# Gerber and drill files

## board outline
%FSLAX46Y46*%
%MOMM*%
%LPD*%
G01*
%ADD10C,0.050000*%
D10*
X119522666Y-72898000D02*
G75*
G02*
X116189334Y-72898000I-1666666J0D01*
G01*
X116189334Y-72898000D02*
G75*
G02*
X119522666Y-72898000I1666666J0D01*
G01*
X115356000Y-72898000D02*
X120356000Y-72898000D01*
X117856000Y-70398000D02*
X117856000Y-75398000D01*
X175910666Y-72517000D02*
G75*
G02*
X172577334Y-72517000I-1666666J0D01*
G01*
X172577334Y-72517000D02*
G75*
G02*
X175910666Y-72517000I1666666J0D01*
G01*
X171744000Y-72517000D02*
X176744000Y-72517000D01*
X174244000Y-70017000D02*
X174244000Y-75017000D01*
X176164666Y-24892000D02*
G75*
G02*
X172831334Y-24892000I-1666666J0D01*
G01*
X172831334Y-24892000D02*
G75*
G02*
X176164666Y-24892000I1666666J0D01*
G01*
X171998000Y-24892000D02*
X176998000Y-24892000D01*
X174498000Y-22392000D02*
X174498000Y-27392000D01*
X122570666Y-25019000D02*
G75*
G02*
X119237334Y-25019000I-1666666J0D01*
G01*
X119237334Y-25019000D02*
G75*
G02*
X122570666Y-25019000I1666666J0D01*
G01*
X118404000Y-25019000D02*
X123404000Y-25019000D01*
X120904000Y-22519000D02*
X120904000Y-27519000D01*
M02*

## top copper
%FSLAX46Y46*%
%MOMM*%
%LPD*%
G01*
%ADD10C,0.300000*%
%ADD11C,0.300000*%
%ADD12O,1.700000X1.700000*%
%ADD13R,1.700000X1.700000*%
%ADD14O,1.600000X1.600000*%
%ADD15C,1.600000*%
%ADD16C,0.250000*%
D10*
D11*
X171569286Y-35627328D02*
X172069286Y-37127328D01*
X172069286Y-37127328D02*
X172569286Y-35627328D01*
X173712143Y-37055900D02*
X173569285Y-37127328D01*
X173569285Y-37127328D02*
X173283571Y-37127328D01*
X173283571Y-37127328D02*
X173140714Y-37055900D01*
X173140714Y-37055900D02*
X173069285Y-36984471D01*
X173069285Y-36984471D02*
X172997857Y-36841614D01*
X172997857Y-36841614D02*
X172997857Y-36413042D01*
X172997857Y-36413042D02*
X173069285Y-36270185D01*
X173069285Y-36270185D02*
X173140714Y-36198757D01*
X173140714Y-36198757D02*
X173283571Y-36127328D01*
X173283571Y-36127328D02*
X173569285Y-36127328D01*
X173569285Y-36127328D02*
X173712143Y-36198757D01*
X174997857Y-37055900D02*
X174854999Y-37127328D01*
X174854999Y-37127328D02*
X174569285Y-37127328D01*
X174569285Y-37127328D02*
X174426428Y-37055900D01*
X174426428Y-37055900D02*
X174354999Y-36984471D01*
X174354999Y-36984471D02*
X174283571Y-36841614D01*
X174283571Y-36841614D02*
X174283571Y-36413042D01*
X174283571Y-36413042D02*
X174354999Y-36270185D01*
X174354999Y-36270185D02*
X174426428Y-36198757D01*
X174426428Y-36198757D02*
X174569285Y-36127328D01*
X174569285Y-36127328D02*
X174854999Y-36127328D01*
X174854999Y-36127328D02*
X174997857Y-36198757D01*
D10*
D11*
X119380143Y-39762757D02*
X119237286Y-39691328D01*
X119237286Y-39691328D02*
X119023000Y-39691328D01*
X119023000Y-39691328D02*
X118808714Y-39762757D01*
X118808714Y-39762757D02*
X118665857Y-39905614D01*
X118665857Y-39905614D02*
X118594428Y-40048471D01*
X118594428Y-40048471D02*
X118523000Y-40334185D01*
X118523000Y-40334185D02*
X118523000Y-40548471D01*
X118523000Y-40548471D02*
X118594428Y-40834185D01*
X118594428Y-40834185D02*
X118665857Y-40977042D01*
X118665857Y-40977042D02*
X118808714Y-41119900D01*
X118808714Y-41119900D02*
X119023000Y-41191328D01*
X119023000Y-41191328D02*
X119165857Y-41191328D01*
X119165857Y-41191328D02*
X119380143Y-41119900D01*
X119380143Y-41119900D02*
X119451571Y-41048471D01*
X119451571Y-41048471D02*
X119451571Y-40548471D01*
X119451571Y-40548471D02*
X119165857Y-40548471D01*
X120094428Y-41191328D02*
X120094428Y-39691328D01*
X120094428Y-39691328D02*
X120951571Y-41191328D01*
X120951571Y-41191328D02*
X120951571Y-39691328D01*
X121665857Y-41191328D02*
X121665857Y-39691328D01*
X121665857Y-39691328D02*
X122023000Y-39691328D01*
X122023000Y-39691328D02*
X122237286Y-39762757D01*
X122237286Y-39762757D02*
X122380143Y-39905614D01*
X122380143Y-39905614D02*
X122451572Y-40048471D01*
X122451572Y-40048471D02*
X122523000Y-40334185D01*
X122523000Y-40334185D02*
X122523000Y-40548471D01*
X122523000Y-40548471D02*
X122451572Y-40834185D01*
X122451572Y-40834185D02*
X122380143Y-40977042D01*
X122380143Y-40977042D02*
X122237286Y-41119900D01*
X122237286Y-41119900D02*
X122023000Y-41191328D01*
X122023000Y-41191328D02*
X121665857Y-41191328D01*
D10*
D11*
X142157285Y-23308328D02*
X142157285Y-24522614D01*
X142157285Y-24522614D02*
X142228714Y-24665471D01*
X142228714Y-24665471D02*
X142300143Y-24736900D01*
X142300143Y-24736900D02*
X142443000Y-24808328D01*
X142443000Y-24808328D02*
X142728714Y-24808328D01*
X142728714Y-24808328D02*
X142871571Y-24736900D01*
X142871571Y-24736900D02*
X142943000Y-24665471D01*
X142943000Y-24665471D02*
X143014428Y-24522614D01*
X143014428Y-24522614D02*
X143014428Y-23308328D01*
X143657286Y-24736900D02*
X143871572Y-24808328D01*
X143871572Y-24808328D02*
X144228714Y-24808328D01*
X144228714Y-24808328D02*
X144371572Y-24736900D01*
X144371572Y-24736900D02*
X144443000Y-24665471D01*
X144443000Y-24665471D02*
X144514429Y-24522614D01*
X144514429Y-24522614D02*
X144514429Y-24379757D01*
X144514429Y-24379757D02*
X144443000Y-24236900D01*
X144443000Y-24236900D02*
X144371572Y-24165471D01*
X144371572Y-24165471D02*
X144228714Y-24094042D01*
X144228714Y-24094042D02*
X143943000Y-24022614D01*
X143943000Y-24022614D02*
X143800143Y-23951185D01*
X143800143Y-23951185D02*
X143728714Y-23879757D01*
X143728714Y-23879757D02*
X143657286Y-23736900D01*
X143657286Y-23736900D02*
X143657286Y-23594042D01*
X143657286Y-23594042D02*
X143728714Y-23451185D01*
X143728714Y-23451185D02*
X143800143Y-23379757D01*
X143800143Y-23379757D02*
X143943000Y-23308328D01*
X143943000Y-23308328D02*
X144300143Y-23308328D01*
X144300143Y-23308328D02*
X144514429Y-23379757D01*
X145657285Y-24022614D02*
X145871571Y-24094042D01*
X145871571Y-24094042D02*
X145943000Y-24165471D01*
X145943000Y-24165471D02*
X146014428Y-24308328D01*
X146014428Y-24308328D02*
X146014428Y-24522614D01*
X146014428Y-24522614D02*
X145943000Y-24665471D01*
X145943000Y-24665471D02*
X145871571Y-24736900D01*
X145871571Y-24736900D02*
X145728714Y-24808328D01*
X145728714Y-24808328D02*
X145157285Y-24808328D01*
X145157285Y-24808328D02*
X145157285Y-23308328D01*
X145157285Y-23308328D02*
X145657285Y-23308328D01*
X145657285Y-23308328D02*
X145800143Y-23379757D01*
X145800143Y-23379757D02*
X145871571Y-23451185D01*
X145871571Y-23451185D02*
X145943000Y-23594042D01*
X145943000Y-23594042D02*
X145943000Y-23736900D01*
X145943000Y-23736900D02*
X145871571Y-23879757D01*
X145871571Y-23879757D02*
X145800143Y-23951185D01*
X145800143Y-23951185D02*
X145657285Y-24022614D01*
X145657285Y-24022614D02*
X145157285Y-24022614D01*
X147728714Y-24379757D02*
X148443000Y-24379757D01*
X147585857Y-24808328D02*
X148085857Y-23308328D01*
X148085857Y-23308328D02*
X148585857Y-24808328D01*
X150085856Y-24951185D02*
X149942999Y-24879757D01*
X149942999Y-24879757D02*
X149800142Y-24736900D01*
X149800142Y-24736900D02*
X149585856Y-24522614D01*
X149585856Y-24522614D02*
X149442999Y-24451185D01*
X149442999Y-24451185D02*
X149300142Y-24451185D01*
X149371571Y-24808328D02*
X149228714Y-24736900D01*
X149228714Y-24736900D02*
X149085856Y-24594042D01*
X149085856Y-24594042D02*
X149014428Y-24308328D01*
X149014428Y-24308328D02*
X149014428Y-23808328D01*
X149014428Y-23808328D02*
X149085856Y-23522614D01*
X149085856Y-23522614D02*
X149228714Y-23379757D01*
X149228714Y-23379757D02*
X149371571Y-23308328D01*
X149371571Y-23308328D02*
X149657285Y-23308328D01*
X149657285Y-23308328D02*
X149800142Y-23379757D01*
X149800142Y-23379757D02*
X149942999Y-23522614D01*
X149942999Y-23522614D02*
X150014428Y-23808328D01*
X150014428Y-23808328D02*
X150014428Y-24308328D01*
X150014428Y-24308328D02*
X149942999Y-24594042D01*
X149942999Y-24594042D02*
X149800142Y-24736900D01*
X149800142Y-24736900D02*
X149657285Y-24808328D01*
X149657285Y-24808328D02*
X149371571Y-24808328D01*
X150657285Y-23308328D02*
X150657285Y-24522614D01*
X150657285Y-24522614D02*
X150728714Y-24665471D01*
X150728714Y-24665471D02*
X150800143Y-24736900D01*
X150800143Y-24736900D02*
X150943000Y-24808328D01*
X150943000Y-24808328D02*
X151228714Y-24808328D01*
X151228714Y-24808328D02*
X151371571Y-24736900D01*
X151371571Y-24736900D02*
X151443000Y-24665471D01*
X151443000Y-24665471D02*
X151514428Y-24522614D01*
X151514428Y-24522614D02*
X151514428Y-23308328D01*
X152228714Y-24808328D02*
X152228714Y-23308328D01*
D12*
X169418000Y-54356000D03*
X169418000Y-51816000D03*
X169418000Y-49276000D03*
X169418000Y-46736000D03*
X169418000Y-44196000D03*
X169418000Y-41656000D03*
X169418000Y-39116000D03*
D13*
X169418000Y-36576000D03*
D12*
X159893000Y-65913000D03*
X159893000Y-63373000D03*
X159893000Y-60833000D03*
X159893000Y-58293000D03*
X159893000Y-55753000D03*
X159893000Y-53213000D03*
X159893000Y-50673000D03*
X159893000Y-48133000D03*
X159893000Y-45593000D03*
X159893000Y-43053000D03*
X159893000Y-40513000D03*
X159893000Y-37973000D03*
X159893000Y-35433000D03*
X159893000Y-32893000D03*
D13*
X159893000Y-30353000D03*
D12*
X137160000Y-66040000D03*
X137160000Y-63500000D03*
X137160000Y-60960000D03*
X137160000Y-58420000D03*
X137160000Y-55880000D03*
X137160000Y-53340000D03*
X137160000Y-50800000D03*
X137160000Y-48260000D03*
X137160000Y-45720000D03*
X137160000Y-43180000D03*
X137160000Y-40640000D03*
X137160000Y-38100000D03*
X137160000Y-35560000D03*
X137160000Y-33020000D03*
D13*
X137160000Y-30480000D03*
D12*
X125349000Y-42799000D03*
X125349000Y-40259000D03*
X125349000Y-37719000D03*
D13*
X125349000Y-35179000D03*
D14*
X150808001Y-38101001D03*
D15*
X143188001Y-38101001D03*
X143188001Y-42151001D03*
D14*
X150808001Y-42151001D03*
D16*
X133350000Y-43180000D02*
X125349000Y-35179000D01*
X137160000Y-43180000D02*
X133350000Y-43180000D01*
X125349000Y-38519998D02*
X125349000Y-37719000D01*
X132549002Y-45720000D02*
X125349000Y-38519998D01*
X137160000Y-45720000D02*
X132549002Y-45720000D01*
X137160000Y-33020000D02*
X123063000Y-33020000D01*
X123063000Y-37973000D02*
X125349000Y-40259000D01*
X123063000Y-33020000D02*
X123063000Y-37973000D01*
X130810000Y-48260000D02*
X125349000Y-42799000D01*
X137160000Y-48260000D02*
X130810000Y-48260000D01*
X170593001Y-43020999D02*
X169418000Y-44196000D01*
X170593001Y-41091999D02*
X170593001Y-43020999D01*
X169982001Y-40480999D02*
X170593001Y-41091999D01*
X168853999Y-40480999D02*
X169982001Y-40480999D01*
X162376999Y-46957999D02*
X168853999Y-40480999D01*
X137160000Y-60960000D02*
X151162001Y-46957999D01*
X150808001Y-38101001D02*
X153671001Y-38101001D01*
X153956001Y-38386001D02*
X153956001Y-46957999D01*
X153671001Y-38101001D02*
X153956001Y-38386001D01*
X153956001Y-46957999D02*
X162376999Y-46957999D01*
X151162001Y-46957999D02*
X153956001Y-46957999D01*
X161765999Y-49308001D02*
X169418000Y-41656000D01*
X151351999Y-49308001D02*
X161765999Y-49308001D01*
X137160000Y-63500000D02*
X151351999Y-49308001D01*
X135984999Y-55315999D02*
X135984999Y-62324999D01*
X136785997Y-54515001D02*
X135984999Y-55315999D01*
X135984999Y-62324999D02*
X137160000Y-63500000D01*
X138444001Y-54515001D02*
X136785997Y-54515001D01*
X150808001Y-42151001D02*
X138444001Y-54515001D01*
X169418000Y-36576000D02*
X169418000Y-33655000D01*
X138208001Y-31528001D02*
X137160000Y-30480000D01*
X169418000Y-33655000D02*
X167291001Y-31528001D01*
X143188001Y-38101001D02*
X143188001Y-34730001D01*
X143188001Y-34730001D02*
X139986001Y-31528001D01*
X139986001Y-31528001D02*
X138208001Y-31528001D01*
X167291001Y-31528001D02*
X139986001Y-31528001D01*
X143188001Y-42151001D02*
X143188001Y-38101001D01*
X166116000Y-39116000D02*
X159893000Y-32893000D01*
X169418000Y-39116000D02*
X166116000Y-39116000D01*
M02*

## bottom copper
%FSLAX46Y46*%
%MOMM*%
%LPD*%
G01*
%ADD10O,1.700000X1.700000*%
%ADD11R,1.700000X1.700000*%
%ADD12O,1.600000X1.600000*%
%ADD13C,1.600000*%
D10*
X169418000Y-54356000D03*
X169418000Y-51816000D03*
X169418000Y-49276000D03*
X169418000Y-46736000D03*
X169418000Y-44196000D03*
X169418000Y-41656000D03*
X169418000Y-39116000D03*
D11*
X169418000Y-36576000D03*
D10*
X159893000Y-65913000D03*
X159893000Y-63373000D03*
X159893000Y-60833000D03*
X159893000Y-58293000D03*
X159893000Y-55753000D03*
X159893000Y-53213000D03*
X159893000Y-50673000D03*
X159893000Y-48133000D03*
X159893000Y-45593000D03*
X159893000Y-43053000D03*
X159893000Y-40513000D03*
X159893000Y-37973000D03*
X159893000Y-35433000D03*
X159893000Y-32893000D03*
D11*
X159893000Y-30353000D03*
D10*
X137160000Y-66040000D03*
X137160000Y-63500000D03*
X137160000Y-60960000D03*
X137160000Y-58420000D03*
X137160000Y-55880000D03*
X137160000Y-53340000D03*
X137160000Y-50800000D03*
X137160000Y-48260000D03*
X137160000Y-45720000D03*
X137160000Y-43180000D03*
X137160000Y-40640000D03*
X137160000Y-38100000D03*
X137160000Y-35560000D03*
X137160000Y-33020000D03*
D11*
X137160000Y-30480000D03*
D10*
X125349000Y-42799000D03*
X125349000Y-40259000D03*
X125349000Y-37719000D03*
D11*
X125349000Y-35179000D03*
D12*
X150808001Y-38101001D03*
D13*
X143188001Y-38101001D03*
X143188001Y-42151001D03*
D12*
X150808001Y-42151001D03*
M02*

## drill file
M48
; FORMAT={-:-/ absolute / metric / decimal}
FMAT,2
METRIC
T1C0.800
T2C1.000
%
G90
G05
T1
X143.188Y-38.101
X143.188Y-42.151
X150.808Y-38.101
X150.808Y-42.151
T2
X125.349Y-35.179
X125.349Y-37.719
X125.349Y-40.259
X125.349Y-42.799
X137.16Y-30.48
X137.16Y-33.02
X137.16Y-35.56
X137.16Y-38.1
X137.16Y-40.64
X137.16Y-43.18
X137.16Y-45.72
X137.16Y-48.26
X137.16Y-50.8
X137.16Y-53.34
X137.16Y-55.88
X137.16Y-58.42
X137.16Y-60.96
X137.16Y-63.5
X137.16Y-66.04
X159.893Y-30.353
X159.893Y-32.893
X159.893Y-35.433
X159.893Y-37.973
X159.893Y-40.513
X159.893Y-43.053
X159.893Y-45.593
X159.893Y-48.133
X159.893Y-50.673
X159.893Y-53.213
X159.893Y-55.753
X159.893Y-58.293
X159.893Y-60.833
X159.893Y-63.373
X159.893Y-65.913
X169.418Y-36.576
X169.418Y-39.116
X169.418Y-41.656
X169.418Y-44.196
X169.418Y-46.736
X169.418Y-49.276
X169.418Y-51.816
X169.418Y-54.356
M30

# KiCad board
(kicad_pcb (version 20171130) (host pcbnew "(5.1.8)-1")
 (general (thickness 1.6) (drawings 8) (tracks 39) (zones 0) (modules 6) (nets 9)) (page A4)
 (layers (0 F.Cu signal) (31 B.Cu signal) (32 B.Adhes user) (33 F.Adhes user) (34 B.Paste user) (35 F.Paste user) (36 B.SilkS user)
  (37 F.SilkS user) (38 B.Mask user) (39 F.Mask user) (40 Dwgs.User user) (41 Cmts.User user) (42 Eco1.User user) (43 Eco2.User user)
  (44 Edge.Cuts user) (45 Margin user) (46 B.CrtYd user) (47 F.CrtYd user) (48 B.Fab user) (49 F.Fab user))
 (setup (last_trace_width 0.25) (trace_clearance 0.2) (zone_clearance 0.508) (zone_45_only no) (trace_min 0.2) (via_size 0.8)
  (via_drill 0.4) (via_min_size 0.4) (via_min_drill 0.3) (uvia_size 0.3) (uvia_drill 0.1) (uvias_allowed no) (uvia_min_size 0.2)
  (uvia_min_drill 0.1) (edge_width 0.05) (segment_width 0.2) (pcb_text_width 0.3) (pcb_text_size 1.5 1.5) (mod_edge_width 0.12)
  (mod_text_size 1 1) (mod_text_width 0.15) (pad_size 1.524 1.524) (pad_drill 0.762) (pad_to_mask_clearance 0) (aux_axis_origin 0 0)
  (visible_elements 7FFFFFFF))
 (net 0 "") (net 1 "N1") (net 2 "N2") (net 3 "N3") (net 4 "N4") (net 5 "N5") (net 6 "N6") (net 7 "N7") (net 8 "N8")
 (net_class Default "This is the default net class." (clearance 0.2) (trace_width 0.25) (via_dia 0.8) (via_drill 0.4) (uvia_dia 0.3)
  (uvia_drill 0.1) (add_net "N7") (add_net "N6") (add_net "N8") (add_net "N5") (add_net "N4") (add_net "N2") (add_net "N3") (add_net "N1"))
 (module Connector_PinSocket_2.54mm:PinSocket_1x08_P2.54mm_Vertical (layer F.Cu) (at 169.418 36.576)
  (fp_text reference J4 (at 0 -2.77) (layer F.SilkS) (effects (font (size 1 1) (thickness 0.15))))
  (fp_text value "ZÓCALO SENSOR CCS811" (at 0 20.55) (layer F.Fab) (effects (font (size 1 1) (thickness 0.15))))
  (pad 8 thru_hole oval (at 0 17.78) (size 1.7 1.7) (drill 1) (layers *.Cu *.Mask))
  (pad 7 thru_hole oval (at 0 15.24) (size 1.7 1.7) (drill 1) (layers *.Cu *.Mask))
  (pad 6 thru_hole oval (at 0 12.7) (size 1.7 1.7) (drill 1) (layers *.Cu *.Mask))
  (pad 5 thru_hole oval (at 0 10.16) (size 1.7 1.7) (drill 1) (layers *.Cu *.Mask) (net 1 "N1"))
  (pad 4 thru_hole oval (at 0 7.62) (size 1.7 1.7) (drill 1) (layers *.Cu *.Mask) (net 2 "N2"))
  (pad 3 thru_hole oval (at 0 5.08) (size 1.7 1.7) (drill 1) (layers *.Cu *.Mask) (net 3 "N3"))
  (pad 2 thru_hole oval (at 0 2.54) (size 1.7 1.7) (drill 1) (layers *.Cu *.Mask) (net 1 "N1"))
  (pad 1 thru_hole rect (at 0 0) (size 1.7 1.7) (drill 1) (layers *.Cu *.Mask) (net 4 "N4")))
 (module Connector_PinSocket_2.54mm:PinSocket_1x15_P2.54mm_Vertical (layer F.Cu) (at 159.893 30.353)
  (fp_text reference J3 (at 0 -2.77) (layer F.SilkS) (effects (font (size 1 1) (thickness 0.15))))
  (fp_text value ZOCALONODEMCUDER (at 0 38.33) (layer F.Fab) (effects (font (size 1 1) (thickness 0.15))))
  (pad 15 thru_hole oval (at 0 35.56) (size 1.7 1.7) (drill 1) (layers *.Cu *.Mask))
  (pad 14 thru_hole oval (at 0 33.02) (size 1.7 1.7) (drill 1) (layers *.Cu *.Mask))
  (pad 13 thru_hole oval (at 0 30.48) (size 1.7 1.7) (drill 1) (layers *.Cu *.Mask))
  (pad 12 thru_hole oval (at 0 27.94) (size 1.7 1.7) (drill 1) (layers *.Cu *.Mask))
  (pad 11 thru_hole oval (at 0 25.4) (size 1.7 1.7) (drill 1) (layers *.Cu *.Mask))
  (pad 10 thru_hole oval (at 0 22.86) (size 1.7 1.7) (drill 1) (layers *.Cu *.Mask))
  (pad 9 thru_hole oval (at 0 20.32) (size 1.7 1.7) (drill 1) (layers *.Cu *.Mask))
  (pad 8 thru_hole oval (at 0 17.78) (size 1.7 1.7) (drill 1) (layers *.Cu *.Mask))
  (pad 7 thru_hole oval (at 0 15.24) (size 1.7 1.7) (drill 1) (layers *.Cu *.Mask))
  (pad 6 thru_hole oval (at 0 12.7) (size 1.7 1.7) (drill 1) (layers *.Cu *.Mask))
  (pad 5 thru_hole oval (at 0 10.16) (size 1.7 1.7) (drill 1) (layers *.Cu *.Mask))
  (pad 4 thru_hole oval (at 0 7.62) (size 1.7 1.7) (drill 1) (layers *.Cu *.Mask))
  (pad 3 thru_hole oval (at 0 5.08) (size 1.7 1.7) (drill 1) (layers *.Cu *.Mask))
  (pad 2 thru_hole oval (at 0 2.54) (size 1.7 1.7) (drill 1) (layers *.Cu *.Mask) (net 1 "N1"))
  (pad 1 thru_hole rect (at 0 0) (size 1.7 1.7) (drill 1) (layers *.Cu *.Mask)))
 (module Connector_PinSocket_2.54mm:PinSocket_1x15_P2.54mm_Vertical (layer F.Cu) (at 137.16 30.48)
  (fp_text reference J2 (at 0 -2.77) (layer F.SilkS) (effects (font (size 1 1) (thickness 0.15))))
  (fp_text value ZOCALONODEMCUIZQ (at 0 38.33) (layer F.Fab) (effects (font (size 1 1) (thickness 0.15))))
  (pad 15 thru_hole oval (at 0 35.56) (size 1.7 1.7) (drill 1) (layers *.Cu *.Mask))
  (pad 14 thru_hole oval (at 0 33.02) (size 1.7 1.7) (drill 1) (layers *.Cu *.Mask) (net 3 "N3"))
  (pad 13 thru_hole oval (at 0 30.48) (size 1.7 1.7) (drill 1) (layers *.Cu *.Mask) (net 2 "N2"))
  (pad 12 thru_hole oval (at 0 27.94) (size 1.7 1.7) (drill 1) (layers *.Cu *.Mask))
  (pad 11 thru_hole oval (at 0 25.4) (size 1.7 1.7) (drill 1) (layers *.Cu *.Mask))
  (pad 10 thru_hole oval (at 0 22.86) (size 1.7 1.7) (drill 1) (layers *.Cu *.Mask))
  (pad 9 thru_hole oval (at 0 20.32) (size 1.7 1.7) (drill 1) (layers *.Cu *.Mask))
  (pad 8 thru_hole oval (at 0 17.78) (size 1.7 1.7) (drill 1) (layers *.Cu *.Mask) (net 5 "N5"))
  (pad 7 thru_hole oval (at 0 15.24) (size 1.7 1.7) (drill 1) (layers *.Cu *.Mask) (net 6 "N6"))
  (pad 6 thru_hole oval (at 0 12.7) (size 1.7 1.7) (drill 1) (layers *.Cu *.Mask) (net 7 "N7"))
  (pad 5 thru_hole oval (at 0 10.16) (size 1.7 1.7) (drill 1) (layers *.Cu *.Mask))
  (pad 4 thru_hole oval (at 0 7.62) (size 1.7 1.7) (drill 1) (layers *.Cu *.Mask))
  (pad 3 thru_hole oval (at 0 5.08) (size 1.7 1.7) (drill 1) (layers *.Cu *.Mask))
  (pad 2 thru_hole oval (at 0 2.54) (size 1.7 1.7) (drill 1) (layers *.Cu *.Mask) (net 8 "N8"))
  (pad 1 thru_hole rect (at 0 0) (size 1.7 1.7) (drill 1) (layers *.Cu *.Mask) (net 4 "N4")))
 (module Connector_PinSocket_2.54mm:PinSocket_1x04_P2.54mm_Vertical (layer F.Cu) (at 125.349 35.179)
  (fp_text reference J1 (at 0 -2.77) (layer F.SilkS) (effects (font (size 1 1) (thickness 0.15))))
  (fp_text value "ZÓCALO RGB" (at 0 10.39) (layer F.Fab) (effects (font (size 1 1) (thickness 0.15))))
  (pad 4 thru_hole oval (at 0 7.62) (size 1.7 1.7) (drill 1) (layers *.Cu *.Mask) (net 5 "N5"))
  (pad 3 thru_hole oval (at 0 5.08) (size 1.7 1.7) (drill 1) (layers *.Cu *.Mask) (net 8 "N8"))
  (pad 2 thru_hole oval (at 0 2.54) (size 1.7 1.7) (drill 1) (layers *.Cu *.Mask) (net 6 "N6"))
  (pad 1 thru_hole rect (at 0 0) (size 1.7 1.7) (drill 1) (layers *.Cu *.Mask) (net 7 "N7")))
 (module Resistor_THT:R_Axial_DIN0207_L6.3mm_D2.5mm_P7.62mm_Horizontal (layer F.Cu) (at 143.188001 38.101001)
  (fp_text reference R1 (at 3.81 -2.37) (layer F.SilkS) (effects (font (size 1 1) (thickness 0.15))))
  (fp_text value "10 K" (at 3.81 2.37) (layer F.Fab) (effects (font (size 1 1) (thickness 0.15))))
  (pad 2 thru_hole oval (at 7.62 0) (size 1.6 1.6) (drill 0.8) (layers *.Cu *.Mask) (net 2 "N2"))
  (pad 1 thru_hole circle (at 0 0) (size 1.6 1.6) (drill 0.8) (layers *.Cu *.Mask) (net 4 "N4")))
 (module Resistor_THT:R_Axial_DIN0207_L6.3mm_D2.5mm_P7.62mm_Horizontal (layer F.Cu) (at 143.188001 42.151001)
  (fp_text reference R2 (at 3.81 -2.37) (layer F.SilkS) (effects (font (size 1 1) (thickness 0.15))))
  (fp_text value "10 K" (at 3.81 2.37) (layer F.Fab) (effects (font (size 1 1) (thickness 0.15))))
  (pad 1 thru_hole circle (at 0 0) (size 1.6 1.6) (drill 0.8) (layers *.Cu *.Mask) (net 4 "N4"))
  (pad 2 thru_hole oval (at 7.62 0) (size 1.6 1.6) (drill 0.8) (layers *.Cu *.Mask) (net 3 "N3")))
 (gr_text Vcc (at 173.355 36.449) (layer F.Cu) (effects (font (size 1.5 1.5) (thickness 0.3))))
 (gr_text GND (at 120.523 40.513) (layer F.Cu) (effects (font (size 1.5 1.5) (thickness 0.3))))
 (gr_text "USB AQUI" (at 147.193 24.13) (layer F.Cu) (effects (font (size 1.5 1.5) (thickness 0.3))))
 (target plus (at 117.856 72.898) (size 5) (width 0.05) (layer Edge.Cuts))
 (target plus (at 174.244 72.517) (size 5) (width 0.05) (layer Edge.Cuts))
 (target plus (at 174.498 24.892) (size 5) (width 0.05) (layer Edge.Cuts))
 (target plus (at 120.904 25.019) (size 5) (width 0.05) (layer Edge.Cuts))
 (segment (start 133.35 43.18) (end 125.349 35.179) (width 0.25) (layer F.Cu) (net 7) (status 20))
 (segment (start 137.16 43.18) (end 133.35 43.18) (width 0.25) (layer F.Cu) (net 7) (status 10))
 (segment (start 125.349 38.519998) (end 125.349 37.719) (width 0.25) (layer F.Cu) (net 6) (status 30))
 (segment (start 132.549002 45.72) (end 125.349 38.519998) (width 0.25) (layer F.Cu) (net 6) (status 20))
 (segment (start 137.16 45.72) (end 132.549002 45.72) (width 0.25) (layer F.Cu) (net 6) (status 10))
 (segment (start 137.16 33.02) (end 123.063 33.02) (width 0.25) (layer F.Cu) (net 8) (status 10))
 (segment (start 123.063 37.973) (end 125.349 40.259) (width 0.25) (layer F.Cu) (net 8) (status 20))
 (segment (start 123.063 33.02) (end 123.063 37.973) (width 0.25) (layer F.Cu) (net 8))
 (segment (start 130.81 48.26) (end 125.349 42.799) (width 0.25) (layer F.Cu) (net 5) (status 20))
 (segment (start 137.16 48.26) (end 130.81 48.26) (width 0.25) (layer F.Cu) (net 5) (status 10))
 (segment (start 170.593001 43.020999) (end 169.418 44.196) (width 0.25) (layer F.Cu) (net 2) (status 20))
 (segment (start 170.593001 41.091999) (end 170.593001 43.020999) (width 0.25) (layer F.Cu) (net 2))
 (segment (start 169.982001 40.480999) (end 170.593001 41.091999) (width 0.25) (layer F.Cu) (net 2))
 (segment (start 168.853999 40.480999) (end 169.982001 40.480999) (width 0.25) (layer F.Cu) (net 2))
 (segment (start 162.376999 46.957999) (end 168.853999 40.480999) (width 0.25) (layer F.Cu) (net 2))
 (segment (start 137.16 60.96) (end 151.162001 46.957999) (width 0.25) (layer F.Cu) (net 2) (status 10))
 (segment (start 150.808001 38.101001) (end 153.671001 38.101001) (width 0.25) (layer F.Cu) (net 2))
 (segment (start 153.956001 38.386001) (end 153.956001 46.957999) (width 0.25) (layer F.Cu) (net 2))
 (segment (start 153.671001 38.101001) (end 153.956001 38.386001) (width 0.25) (layer F.Cu) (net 2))
 (segment (start 153.956001 46.957999) (end 162.376999 46.957999) (width 0.25) (layer F.Cu) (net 2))
 (segment (start 151.162001 46.957999) (end 153.956001 46.957999) (width 0.25) (layer F.Cu) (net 2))
 (segment (start 161.765999 49.308001) (end 169.418 41.656) (width 0.25) (layer F.Cu) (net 3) (status 20))
 (segment (start 151.351999 49.308001) (end 161.765999 49.308001) (width 0.25) (layer F.Cu) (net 3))
 (segment (start 137.16 63.5) (end 151.351999 49.308001) (width 0.25) (layer F.Cu) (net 3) (status 10))
 (segment (start 135.984999 55.315999) (end 135.984999 62.324999) (width 0.25) (layer F.Cu) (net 3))
 (segment (start 136.785997 54.515001) (end 135.984999 55.315999) (width 0.25) (layer F.Cu) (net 3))
 (segment (start 135.984999 62.324999) (end 137.16 63.5) (width 0.25) (layer F.Cu) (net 3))
 (segment (start 138.444001 54.515001) (end 136.785997 54.515001) (width 0.25) (layer F.Cu) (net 3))
 (segment (start 150.808001 42.151001) (end 138.444001 54.515001) (width 0.25) (layer F.Cu) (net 3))
 (segment (start 169.418 36.576) (end 169.418 33.655) (width 0.25) (layer F.Cu) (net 4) (status 10))
 (segment (start 138.208001 31.528001) (end 137.16 30.48) (width 0.25) (layer F.Cu) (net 4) (status 20))
 (segment (start 169.418 33.655) (end 167.291001 31.528001) (width 0.25) (layer F.Cu) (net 4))
 (segment (start 143.188001 38.101001) (end 143.188001 34.730001) (width 0.25) (layer F.Cu) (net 4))
 (segment (start 143.188001 34.730001) (end 139.986001 31.528001) (width 0.25) (layer F.Cu) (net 4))
 (segment (start 139.986001 31.528001) (end 138.208001 31.528001) (width 0.25) (layer F.Cu) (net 4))
 (segment (start 167.291001 31.528001) (end 139.986001 31.528001) (width 0.25) (layer F.Cu) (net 4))
 (segment (start 143.188001 42.151001) (end 143.188001 38.101001) (width 0.25) (layer F.Cu) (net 4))
 (segment (start 166.116 39.116) (end 159.893 32.893) (width 0.25) (layer F.Cu) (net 1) (status 20))
 (segment (start 169.418 39.116) (end 166.116 39.116) (width 0.25) (layer F.Cu) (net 1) (status 10)))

